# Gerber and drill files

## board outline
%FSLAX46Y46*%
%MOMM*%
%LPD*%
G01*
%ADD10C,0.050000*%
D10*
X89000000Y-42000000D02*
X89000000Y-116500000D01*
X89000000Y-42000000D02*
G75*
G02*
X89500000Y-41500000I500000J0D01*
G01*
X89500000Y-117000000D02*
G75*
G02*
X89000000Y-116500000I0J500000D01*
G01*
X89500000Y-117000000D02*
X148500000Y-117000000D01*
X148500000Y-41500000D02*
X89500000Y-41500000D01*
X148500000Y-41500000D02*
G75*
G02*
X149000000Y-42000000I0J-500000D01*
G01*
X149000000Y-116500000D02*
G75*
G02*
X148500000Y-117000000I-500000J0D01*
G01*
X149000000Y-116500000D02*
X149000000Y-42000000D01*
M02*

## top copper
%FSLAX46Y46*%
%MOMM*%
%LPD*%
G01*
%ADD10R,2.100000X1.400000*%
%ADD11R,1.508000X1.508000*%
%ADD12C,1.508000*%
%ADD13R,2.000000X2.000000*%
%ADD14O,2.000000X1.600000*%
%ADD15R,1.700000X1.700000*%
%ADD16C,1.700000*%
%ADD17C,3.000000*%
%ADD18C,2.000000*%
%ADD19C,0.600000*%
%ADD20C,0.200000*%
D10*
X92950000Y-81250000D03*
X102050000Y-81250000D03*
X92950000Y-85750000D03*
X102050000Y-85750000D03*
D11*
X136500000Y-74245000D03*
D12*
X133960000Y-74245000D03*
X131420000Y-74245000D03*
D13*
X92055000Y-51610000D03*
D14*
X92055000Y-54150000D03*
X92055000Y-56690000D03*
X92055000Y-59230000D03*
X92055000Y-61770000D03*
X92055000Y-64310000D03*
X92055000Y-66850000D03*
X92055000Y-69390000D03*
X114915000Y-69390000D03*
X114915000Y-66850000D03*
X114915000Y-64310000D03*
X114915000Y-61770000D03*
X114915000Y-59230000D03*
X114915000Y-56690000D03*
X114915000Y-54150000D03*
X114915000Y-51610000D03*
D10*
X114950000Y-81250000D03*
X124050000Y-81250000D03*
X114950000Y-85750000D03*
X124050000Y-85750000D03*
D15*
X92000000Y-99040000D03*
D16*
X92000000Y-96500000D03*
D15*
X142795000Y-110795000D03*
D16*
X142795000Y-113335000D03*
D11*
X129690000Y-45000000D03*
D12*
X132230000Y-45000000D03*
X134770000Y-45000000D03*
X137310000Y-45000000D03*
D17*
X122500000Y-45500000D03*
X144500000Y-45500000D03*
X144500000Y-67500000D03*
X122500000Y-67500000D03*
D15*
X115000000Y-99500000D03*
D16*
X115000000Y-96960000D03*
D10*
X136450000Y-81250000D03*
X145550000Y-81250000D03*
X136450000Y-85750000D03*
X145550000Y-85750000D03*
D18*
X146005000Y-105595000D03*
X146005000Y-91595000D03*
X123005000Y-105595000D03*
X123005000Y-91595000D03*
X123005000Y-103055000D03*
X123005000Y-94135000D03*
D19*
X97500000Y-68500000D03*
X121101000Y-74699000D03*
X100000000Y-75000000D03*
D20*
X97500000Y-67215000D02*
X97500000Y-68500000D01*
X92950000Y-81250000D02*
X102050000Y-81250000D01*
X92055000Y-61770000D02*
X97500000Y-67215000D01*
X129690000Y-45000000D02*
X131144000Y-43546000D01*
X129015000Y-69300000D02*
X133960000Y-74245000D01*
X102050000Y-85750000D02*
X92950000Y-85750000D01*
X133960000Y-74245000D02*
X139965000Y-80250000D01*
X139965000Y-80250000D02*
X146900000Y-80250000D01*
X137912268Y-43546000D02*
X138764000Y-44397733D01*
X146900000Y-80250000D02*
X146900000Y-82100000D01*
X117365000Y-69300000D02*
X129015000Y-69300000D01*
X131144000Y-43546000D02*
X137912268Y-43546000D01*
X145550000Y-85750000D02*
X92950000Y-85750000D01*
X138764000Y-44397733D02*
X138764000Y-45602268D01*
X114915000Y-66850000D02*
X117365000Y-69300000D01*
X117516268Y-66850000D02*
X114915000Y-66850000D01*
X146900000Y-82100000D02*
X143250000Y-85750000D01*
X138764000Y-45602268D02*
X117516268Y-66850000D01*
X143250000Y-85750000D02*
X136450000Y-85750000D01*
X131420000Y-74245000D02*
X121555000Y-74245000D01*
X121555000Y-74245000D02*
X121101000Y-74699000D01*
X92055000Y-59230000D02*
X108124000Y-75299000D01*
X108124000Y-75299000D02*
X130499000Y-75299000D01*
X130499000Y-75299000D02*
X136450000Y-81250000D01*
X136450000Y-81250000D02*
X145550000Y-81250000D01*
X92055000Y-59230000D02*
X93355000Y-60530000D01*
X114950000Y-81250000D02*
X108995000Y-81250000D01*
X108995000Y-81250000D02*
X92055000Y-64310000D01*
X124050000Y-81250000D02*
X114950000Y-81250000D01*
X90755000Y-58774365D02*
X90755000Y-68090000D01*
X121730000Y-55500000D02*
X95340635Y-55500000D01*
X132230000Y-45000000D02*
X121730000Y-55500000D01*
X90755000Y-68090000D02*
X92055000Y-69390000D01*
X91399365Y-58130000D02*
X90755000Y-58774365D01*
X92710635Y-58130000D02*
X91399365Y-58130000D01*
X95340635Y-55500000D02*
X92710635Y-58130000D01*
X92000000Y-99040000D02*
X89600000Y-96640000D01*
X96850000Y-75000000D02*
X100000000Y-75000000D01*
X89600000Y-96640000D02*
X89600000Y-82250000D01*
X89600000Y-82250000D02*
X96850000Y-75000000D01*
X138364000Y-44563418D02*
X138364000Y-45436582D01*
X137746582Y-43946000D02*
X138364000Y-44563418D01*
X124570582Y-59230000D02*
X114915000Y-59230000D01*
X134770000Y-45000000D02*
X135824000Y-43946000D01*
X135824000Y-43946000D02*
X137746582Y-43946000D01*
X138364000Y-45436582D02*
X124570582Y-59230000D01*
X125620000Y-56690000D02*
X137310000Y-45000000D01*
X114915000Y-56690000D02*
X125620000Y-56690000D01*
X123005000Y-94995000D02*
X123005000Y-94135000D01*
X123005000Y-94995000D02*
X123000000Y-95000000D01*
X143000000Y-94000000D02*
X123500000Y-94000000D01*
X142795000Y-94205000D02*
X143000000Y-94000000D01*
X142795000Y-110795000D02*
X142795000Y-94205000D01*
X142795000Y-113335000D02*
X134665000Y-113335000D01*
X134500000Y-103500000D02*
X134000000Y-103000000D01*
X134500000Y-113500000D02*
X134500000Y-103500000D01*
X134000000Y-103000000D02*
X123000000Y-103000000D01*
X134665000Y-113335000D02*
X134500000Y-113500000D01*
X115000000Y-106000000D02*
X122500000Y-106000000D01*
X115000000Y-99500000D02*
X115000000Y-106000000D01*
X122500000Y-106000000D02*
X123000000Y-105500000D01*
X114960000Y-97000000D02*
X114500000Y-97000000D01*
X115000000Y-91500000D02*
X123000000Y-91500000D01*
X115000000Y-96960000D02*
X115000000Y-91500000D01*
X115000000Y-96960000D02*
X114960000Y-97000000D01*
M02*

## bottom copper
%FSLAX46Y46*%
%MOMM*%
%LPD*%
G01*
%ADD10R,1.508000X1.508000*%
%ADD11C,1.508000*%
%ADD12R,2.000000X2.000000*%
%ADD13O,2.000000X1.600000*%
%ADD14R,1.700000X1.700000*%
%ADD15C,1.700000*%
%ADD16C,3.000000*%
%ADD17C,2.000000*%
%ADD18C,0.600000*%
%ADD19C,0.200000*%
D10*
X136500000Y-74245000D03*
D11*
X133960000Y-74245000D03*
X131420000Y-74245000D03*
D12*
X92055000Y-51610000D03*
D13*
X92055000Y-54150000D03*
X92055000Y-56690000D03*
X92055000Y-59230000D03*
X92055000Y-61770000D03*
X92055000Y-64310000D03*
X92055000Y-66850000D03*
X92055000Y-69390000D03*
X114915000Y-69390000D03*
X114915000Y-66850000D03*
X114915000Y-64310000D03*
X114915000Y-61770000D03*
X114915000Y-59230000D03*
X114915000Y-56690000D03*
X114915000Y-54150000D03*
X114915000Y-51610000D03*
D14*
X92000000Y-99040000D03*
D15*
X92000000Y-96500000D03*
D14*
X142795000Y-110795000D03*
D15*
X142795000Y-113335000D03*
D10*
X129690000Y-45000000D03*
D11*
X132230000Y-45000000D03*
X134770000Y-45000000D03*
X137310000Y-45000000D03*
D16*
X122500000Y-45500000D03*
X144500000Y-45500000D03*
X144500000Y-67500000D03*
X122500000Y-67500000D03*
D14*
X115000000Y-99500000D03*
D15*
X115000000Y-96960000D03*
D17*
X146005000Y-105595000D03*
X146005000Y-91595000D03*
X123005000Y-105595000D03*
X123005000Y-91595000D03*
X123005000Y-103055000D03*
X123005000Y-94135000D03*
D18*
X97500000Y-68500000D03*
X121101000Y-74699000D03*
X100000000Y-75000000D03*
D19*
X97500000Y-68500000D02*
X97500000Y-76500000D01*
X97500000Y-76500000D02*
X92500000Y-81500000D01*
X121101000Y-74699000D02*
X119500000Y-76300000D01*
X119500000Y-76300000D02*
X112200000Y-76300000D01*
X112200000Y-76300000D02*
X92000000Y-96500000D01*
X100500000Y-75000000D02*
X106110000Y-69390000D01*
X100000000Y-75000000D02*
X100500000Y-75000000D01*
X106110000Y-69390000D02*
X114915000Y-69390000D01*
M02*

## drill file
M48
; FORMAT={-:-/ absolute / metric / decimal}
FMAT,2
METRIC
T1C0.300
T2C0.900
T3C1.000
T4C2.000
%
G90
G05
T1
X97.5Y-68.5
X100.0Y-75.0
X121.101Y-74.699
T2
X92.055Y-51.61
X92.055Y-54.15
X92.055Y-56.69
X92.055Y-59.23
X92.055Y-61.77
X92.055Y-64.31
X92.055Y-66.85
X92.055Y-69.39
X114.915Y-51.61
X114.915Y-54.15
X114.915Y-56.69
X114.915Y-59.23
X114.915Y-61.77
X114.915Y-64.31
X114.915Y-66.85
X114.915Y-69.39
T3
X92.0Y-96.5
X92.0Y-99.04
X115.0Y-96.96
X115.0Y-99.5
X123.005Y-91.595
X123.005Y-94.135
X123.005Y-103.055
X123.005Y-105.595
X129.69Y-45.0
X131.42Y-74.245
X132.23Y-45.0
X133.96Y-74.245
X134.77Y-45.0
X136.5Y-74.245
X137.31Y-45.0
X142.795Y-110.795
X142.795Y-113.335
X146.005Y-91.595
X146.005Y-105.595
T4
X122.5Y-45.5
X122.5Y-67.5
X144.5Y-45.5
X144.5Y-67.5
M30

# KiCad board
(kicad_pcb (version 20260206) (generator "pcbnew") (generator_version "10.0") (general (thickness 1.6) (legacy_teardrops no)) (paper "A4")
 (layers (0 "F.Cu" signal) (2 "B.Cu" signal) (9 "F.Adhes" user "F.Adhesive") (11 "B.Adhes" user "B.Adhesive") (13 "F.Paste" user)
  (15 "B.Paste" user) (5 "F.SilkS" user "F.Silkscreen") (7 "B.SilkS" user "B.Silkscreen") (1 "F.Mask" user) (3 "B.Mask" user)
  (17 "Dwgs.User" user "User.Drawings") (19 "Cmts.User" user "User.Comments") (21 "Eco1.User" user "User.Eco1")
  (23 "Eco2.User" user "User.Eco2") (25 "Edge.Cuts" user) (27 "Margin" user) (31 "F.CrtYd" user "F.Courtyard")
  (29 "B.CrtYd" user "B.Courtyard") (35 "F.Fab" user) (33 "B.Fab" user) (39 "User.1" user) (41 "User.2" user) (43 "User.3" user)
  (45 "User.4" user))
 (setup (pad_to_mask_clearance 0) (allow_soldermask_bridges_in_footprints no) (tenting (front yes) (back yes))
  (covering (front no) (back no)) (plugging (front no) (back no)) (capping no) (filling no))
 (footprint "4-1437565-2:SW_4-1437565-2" (layer "F.Cu") (at 97.5 83.5)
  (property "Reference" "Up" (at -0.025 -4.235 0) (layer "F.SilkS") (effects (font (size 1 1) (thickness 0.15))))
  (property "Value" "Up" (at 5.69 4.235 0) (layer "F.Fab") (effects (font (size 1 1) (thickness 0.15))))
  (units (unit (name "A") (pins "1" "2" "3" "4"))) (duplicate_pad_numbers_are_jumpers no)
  (pad "1" smd rect (at -4.55 -2.25) (size 2.1 1.4) (layers "F.Cu" "F.Mask" "F.Paste") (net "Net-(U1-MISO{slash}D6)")
   (solder_mask_margin 0.102))
  (pad "2" smd rect (at 4.55 -2.25) (size 2.1 1.4) (layers "F.Cu" "F.Mask" "F.Paste") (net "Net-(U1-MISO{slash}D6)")
   (solder_mask_margin 0.102))
  (pad "3" smd rect (at -4.55 2.25) (size 2.1 1.4) (layers "F.Cu" "F.Mask" "F.Paste") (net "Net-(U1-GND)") (solder_mask_margin 0.102))
  (pad "4" smd rect (at 4.55 2.25) (size 2.1 1.4) (layers "F.Cu" "F.Mask" "F.Paste") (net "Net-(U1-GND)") (solder_mask_margin 0.102)))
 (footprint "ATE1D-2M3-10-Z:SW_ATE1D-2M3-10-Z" (layer "F.Cu") (at 133.96 74.245)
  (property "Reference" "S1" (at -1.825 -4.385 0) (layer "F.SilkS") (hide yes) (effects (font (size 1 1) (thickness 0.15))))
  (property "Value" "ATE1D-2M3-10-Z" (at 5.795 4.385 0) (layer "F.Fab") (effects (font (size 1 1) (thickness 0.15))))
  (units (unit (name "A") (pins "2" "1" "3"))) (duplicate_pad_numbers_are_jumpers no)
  (pad "1" thru_hole rect (at 2.54 0) (size 1.508 1.508) (drill 1) (layers "*.Cu" "*.Mask") (remove_unused_layers no)
   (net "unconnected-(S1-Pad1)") (solder_mask_margin 0.102))
  (pad "2" thru_hole circle (at 0 0) (size 1.508 1.508) (drill 1) (layers "*.Cu" "*.Mask") (remove_unused_layers no) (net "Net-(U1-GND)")
   (solder_mask_margin 0.102))
  (pad "3" thru_hole circle (at -2.54 0) (size 1.508 1.508) (drill 1) (layers "*.Cu" "*.Mask") (remove_unused_layers no)
   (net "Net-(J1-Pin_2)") (solder_mask_margin 0.102)))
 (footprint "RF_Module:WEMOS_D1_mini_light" (layer "F.Cu") (at 92.055 51.61)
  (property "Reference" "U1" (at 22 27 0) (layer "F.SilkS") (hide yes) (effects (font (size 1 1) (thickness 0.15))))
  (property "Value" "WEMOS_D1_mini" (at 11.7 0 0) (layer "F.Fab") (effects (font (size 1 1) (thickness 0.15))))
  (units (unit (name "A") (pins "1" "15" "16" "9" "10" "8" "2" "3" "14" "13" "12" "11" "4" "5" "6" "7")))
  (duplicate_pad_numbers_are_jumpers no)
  (pad "1" thru_hole rect (at 0 0) (size 2 2) (drill 0.9) (layers "*.Cu" "*.Mask") (remove_unused_layers no)
   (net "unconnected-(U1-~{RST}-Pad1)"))
  (pad "2" thru_hole oval (at 0 2.54) (size 2 1.6) (drill 0.9) (layers "*.Cu" "*.Mask") (remove_unused_layers no)
   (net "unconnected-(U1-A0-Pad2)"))
  (pad "3" thru_hole oval (at 0 5.08) (size 2 1.6) (drill 0.9) (layers "*.Cu" "*.Mask") (remove_unused_layers no)
   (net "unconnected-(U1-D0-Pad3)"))
  (pad "4" thru_hole oval (at 0 7.62) (size 2 1.6) (drill 0.9) (layers "*.Cu" "*.Mask") (remove_unused_layers no)
   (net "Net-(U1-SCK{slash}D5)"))
  (pad "5" thru_hole oval (at 0 10.16) (size 2 1.6) (drill 0.9) (layers "*.Cu" "*.Mask") (remove_unused_layers no)
   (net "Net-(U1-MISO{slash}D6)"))
  (pad "6" thru_hole oval (at 0 12.7) (size 2 1.6) (drill 0.9) (layers "*.Cu" "*.Mask") (remove_unused_layers no)
   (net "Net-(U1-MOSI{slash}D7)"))
  (pad "7" thru_hole oval (at 0 15.24) (size 2 1.6) (drill 0.9) (layers "*.Cu" "*.Mask") (remove_unused_layers no)
   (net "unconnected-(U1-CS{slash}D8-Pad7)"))
  (pad "8" thru_hole oval (at 0 17.78) (size 2 1.6) (drill 0.9) (layers "*.Cu" "*.Mask") (remove_unused_layers no) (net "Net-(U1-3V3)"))
  (pad "9" thru_hole oval (at 22.86 17.78) (size 2 1.6) (drill 0.9) (layers "*.Cu" "*.Mask") (remove_unused_layers no)
   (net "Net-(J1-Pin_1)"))
  (pad "10" thru_hole oval (at 22.86 15.24) (size 2 1.6) (drill 0.9) (layers "*.Cu" "*.Mask") (remove_unused_layers no) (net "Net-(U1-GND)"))
  (pad "11" thru_hole oval (at 22.86 12.7) (size 2 1.6) (drill 0.9) (layers "*.Cu" "*.Mask") (remove_unused_layers no)
   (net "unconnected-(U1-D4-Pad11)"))
  (pad "12" thru_hole oval (at 22.86 10.16) (size 2 1.6) (drill 0.9) (layers "*.Cu" "*.Mask") (remove_unused_layers no)
   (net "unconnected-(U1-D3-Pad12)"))
  (pad "13" thru_hole oval (at 22.86 7.62) (size 2 1.6) (drill 0.9) (layers "*.Cu" "*.Mask") (remove_unused_layers no)
   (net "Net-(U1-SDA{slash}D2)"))
  (pad "14" thru_hole oval (at 22.86 5.08) (size 2 1.6) (drill 0.9) (layers "*.Cu" "*.Mask") (remove_unused_layers no)
   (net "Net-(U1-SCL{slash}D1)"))
  (pad "15" thru_hole oval (at 22.86 2.54) (size 2 1.6) (drill 0.9) (layers "*.Cu" "*.Mask") (remove_unused_layers no)
   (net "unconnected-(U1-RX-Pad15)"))
  (pad "16" thru_hole oval (at 22.86 0) (size 2 1.6) (drill 0.9) (layers "*.Cu" "*.Mask") (remove_unused_layers no)
   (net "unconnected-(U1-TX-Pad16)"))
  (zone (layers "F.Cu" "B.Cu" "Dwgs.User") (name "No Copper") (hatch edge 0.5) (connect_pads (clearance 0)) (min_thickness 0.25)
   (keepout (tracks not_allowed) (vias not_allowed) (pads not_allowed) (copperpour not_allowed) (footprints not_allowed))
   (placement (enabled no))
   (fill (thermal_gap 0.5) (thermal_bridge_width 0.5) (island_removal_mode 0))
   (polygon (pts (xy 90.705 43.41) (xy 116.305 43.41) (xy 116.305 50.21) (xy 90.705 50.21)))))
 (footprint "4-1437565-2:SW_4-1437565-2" (layer "F.Cu") (at 119.5 83.5)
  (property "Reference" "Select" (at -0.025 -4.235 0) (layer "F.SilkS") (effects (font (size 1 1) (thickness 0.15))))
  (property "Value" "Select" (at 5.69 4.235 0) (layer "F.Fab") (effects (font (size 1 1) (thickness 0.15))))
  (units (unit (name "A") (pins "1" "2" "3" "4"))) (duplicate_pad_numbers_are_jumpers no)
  (pad "1" smd rect (at -4.55 -2.25) (size 2.1 1.4) (layers "F.Cu" "F.Mask" "F.Paste") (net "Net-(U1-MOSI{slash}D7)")
   (solder_mask_margin 0.102))
  (pad "2" smd rect (at 4.55 -2.25) (size 2.1 1.4) (layers "F.Cu" "F.Mask" "F.Paste") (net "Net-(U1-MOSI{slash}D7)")
   (solder_mask_margin 0.102))
  (pad "3" smd rect (at -4.55 2.25) (size 2.1 1.4) (layers "F.Cu" "F.Mask" "F.Paste") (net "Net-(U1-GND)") (solder_mask_margin 0.102))
  (pad "4" smd rect (at 4.55 2.25) (size 2.1 1.4) (layers "F.Cu" "F.Mask" "F.Paste") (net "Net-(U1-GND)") (solder_mask_margin 0.102)))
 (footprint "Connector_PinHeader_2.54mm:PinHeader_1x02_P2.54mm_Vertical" (layer "F.Cu") (at 92 99.04 180)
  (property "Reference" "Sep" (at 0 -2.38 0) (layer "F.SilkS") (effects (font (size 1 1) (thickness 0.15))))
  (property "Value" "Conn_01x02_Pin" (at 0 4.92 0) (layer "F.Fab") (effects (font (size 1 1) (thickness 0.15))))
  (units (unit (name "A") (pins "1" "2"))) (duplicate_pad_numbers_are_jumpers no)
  (pad "1" thru_hole rect (at 0 0 180) (size 1.7 1.7) (drill 1) (layers "*.Cu" "*.Mask") (remove_unused_layers no) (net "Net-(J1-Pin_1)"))
  (pad "2" thru_hole circle (at 0 2.54 180) (size 1.7 1.7) (drill 1) (layers "*.Cu" "*.Mask") (remove_unused_layers no)
   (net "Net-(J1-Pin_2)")))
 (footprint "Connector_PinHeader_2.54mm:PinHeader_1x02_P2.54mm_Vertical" (layer "F.Cu") (at 142.795 110.795)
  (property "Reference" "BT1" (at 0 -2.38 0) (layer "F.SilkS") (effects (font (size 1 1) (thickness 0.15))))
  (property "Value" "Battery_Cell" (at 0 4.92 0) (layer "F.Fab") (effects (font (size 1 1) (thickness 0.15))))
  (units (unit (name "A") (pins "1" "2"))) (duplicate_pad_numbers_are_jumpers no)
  (pad "1" thru_hole rect (at 0 0) (size 1.7 1.7) (drill 1) (layers "*.Cu" "*.Mask") (remove_unused_layers no)
   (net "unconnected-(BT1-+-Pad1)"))
  (pad "2" thru_hole circle (at 0 2.54) (size 1.7 1.7) (drill 1) (layers "*.Cu" "*.Mask") (remove_unused_layers no)
   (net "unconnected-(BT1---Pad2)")))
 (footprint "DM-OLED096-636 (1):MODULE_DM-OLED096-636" (layer "F.Cu") (at 133.5 56.5)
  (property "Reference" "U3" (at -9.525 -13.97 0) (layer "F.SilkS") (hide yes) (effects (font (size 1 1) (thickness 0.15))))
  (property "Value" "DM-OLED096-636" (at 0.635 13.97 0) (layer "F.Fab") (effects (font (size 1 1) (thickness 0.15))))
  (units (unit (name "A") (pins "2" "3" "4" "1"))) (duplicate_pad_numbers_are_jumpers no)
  (pad "1" thru_hole rect (at -3.81 -11.5) (size 1.508 1.508) (drill 1) (layers "*.Cu" "*.Mask") (remove_unused_layers no)
   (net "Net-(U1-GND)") (solder_mask_margin 0.102))
  (pad "2" thru_hole circle (at -1.27 -11.5) (size 1.508 1.508) (drill 1) (layers "*.Cu" "*.Mask") (remove_unused_layers no)
   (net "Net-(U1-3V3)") (solder_mask_margin 0.102))
  (pad "3" thru_hole circle (at 1.27 -11.5) (size 1.508 1.508) (drill 1) (layers "*.Cu" "*.Mask") (remove_unused_layers no)
   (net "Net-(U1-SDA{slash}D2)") (solder_mask_margin 0.102))
  (pad "4" thru_hole circle (at 3.81 -11.5) (size 1.508 1.508) (drill 1) (layers "*.Cu" "*.Mask") (remove_unused_layers no)
   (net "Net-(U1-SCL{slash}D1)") (solder_mask_margin 0.102))
  (pad "S1" thru_hole circle (at -11 -11) (size 3 3) (drill 2) (layers "*.Cu" "*.Mask") (remove_unused_layers no) (solder_mask_margin 0.102))
  (pad "S2" thru_hole circle (at 11 -11) (size 3 3) (drill 2) (layers "*.Cu" "*.Mask") (remove_unused_layers no) (solder_mask_margin 0.102))
  (pad "S3" thru_hole circle (at 11 11) (size 3 3) (drill 2) (layers "*.Cu" "*.Mask") (remove_unused_layers no) (solder_mask_margin 0.102))
  (pad "S4" thru_hole circle (at -11 11) (size 3 3) (drill 2) (layers "*.Cu" "*.Mask") (remove_unused_layers no) (solder_mask_margin 0.102)))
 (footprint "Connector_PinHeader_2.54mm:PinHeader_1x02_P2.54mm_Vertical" (layer "F.Cu") (at 115 99.5 180)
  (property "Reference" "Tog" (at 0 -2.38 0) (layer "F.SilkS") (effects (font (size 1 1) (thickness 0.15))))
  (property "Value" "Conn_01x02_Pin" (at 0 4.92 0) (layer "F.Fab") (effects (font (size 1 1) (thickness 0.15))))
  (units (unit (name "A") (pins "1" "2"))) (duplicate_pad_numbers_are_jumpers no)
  (pad "1" thru_hole rect (at 0 0 180) (size 1.7 1.7) (drill 1) (layers "*.Cu" "*.Mask") (remove_unused_layers no)
   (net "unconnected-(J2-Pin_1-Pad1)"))
  (pad "2" thru_hole circle (at 0 2.54 180) (size 1.7 1.7) (drill 1) (layers "*.Cu" "*.Mask") (remove_unused_layers no)
   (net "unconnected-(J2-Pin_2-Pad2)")))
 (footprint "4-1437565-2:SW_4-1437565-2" (layer "F.Cu") (at 141 83.5)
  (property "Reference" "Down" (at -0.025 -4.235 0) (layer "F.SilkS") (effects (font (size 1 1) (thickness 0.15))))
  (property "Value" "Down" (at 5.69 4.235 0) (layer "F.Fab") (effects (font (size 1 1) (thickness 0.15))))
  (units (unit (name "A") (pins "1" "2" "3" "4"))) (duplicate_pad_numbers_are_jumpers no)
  (pad "1" smd rect (at -4.55 -2.25) (size 2.1 1.4) (layers "F.Cu" "F.Mask" "F.Paste") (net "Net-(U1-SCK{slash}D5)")
   (solder_mask_margin 0.102))
  (pad "2" smd rect (at 4.55 -2.25) (size 2.1 1.4) (layers "F.Cu" "F.Mask" "F.Paste") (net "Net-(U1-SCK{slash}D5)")
   (solder_mask_margin 0.102))
  (pad "3" smd rect (at -4.55 2.25) (size 2.1 1.4) (layers "F.Cu" "F.Mask" "F.Paste") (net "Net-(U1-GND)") (solder_mask_margin 0.102))
  (pad "4" smd rect (at 4.55 2.25) (size 2.1 1.4) (layers "F.Cu" "F.Mask" "F.Paste") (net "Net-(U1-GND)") (solder_mask_margin 0.102)))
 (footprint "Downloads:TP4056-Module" (layer "F.Cu") (at 148.505 89.995 180)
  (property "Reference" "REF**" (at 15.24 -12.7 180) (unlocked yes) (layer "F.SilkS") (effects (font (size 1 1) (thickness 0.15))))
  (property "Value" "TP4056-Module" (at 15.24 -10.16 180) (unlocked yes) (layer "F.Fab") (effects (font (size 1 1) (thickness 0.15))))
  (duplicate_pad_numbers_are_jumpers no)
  (pad "1" thru_hole circle (at 2.5 -15.6 180) (size 2 2) (drill 1) (layers "*.Cu" "*.Mask") (remove_unused_layers no))
  (pad "2" thru_hole circle (at 2.5 -1.6 180) (size 2 2) (drill 1) (layers "*.Cu" "*.Mask") (remove_unused_layers no))
  (pad "3" thru_hole circle (at 25.5 -15.6 180) (size 2 2) (drill 1) (layers "*.Cu" "*.Mask") (remove_unused_layers no))
  (pad "4" thru_hole circle (at 25.5 -1.6 180) (size 2 2) (drill 1) (layers "*.Cu" "*.Mask") (remove_unused_layers no))
  (pad "5" thru_hole circle (at 25.5 -13.06 180) (size 2 2) (drill 1) (layers "*.Cu" "*.Mask") (remove_unused_layers no))
  (pad "6" thru_hole circle (at 25.5 -4.14 180) (size 2 2) (drill 1) (layers "*.Cu" "*.Mask") (remove_unused_layers no)))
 (gr_line (start 89 42) (end 89 116.5) (stroke (width 0.05) (type default)) (layer "Edge.Cuts"))
 (gr_arc (start 89 42) (mid 89.146447 41.646447) (end 89.5 41.5) (stroke (width 0.05) (type default)) (layer "Edge.Cuts"))
 (gr_arc (start 89.5 117) (mid 89.146447 116.853553) (end 89 116.5) (stroke (width 0.05) (type default)) (layer "Edge.Cuts"))
 (gr_line (start 89.5 117) (end 148.5 117) (stroke (width 0.05) (type default)) (layer "Edge.Cuts"))
 (gr_line (start 148.5 41.5) (end 89.5 41.5) (stroke (width 0.05) (type default)) (layer "Edge.Cuts"))
 (gr_arc (start 148.5 41.5) (mid 148.853553 41.646447) (end 149 42) (stroke (width 0.05) (type default)) (layer "Edge.Cuts"))
 (gr_arc (start 149 116.5) (mid 148.853553 116.853553) (end 148.5 117) (stroke (width 0.05) (type default)) (layer "Edge.Cuts"))
 (gr_line (start 149 116.5) (end 149 42) (stroke (width 0.05) (type default)) (layer "Edge.Cuts"))
 (segment (start 97.5 67.215) (end 97.5 68.5) (width 0.2) (layer "F.Cu") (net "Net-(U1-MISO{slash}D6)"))
 (segment (start 92.95 81.25) (end 102.05 81.25) (width 0.2) (layer "F.Cu") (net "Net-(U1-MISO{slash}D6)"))
 (segment (start 92.055 61.77) (end 97.5 67.215) (width 0.2) (layer "F.Cu") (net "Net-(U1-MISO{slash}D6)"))
 (via (at 97.5 68.5) (size 0.6) (drill 0.3) (layers "F.Cu" "B.Cu") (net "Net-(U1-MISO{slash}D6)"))
 (segment (start 97.5 68.5) (end 97.5 76.5) (width 0.2) (layer "B.Cu") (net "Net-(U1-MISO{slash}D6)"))
 (segment (start 97.5 76.5) (end 92.5 81.5) (width 0.2) (layer "B.Cu") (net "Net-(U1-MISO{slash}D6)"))
 (segment (start 129.69 45) (end 131.144 43.546) (width 0.2) (layer "F.Cu") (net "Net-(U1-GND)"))
 (segment (start 129.015 69.3) (end 133.96 74.245) (width 0.2) (layer "F.Cu") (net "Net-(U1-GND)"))
 (segment (start 102.05 85.75) (end 92.95 85.75) (width 0.2) (layer "F.Cu") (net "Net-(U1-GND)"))
 (segment (start 133.96 74.245) (end 139.965 80.25) (width 0.2) (layer "F.Cu") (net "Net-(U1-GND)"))
 (segment (start 139.965 80.25) (end 146.9 80.25) (width 0.2) (layer "F.Cu") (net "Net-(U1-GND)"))
 (segment (start 137.912268 43.546) (end 138.764 44.397733) (width 0.2) (layer "F.Cu") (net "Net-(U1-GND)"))
 (segment (start 146.9 80.25) (end 146.9 82.1) (width 0.2) (layer "F.Cu") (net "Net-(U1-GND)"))
 (segment (start 117.365 69.3) (end 129.015 69.3) (width 0.2) (layer "F.Cu") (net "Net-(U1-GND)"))
 (segment (start 131.144 43.546) (end 137.912268 43.546) (width 0.2) (layer "F.Cu") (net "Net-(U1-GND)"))
 (segment (start 145.55 85.75) (end 92.95 85.75) (width 0.2) (layer "F.Cu") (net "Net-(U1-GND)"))
 (segment (start 138.764 44.397733) (end 138.764 45.602268) (width 0.2) (layer "F.Cu") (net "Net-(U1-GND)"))
 (segment (start 114.915 66.85) (end 117.365 69.3) (width 0.2) (layer "F.Cu") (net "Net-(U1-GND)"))
 (segment (start 117.516268 66.85) (end 114.915 66.85) (width 0.2) (layer "F.Cu") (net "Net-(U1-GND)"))
 (segment (start 146.9 82.1) (end 143.25 85.75) (width 0.2) (layer "F.Cu") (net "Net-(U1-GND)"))
 (segment (start 138.764 45.602268) (end 117.516268 66.85) (width 0.2) (layer "F.Cu") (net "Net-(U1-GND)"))
 (segment (start 143.25 85.75) (end 136.45 85.75) (width 0.2) (layer "F.Cu") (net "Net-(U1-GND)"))
 (segment (start 131.42 74.245) (end 121.555 74.245) (width 0.2) (layer "F.Cu") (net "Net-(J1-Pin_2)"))
 (segment (start 121.555 74.245) (end 121.101 74.699) (width 0.2) (layer "F.Cu") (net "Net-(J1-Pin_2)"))
 (via (at 121.101 74.699) (size 0.6) (drill 0.3) (layers "F.Cu" "B.Cu") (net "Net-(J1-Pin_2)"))
 (segment (start 121.101 74.699) (end 119.5 76.3) (width 0.2) (layer "B.Cu") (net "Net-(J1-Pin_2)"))
 (segment (start 119.5 76.3) (end 112.2 76.3) (width 0.2) (layer "B.Cu") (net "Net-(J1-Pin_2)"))
 (segment (start 112.2 76.3) (end 92 96.5) (width 0.2) (layer "B.Cu") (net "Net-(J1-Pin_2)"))
 (segment (start 92.055 59.23) (end 108.124 75.299) (width 0.2) (layer "F.Cu") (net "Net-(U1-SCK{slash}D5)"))
 (segment (start 108.124 75.299) (end 130.499 75.299) (width 0.2) (layer "F.Cu") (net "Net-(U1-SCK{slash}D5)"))
 (segment (start 130.499 75.299) (end 136.45 81.25) (width 0.2) (layer "F.Cu") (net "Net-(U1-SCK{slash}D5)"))
 (segment (start 136.45 81.25) (end 145.55 81.25) (width 0.2) (layer "F.Cu") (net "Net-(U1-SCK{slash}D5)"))
 (segment (start 92.055 59.23) (end 93.355 60.53) (width 0.2) (layer "F.Cu") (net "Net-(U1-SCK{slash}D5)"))
 (segment (start 114.95 81.25) (end 108.995 81.25) (width 0.2) (layer "F.Cu") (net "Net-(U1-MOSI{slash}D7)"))
 (segment (start 108.995 81.25) (end 92.055 64.31) (width 0.2) (layer "F.Cu") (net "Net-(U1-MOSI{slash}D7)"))
 (segment (start 124.05 81.25) (end 114.95 81.25) (width 0.2) (layer "F.Cu") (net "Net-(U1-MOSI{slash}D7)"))
 (segment (start 90.755 58.774365) (end 90.755 68.09) (width 0.2) (layer "F.Cu") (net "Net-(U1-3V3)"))
 (segment (start 121.73 55.5) (end 95.340635 55.5) (width 0.2) (layer "F.Cu") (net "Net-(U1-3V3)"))
 (segment (start 132.23 45) (end 121.73 55.5) (width 0.2) (layer "F.Cu") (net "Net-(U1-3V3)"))
 (segment (start 90.755 68.09) (end 92.055 69.39) (width 0.2) (layer "F.Cu") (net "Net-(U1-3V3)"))
 (segment (start 91.399365 58.13) (end 90.755 58.774365) (width 0.2) (layer "F.Cu") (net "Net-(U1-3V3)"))
 (segment (start 92.710635 58.13) (end 91.399365 58.13) (width 0.2) (layer "F.Cu") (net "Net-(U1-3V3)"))
 (segment (start 95.340635 55.5) (end 92.710635 58.13) (width 0.2) (layer "F.Cu") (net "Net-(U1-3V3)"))
 (segment (start 92 99.04) (end 89.6 96.64) (width 0.2) (layer "F.Cu") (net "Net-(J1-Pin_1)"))
 (segment (start 96.85 75) (end 100 75) (width 0.2) (layer "F.Cu") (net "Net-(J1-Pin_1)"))
 (segment (start 89.6 96.64) (end 89.6 82.25) (width 0.2) (layer "F.Cu") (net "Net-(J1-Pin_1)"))
 (segment (start 89.6 82.25) (end 96.85 75) (width 0.2) (layer "F.Cu") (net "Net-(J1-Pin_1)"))
 (via (at 100 75) (size 0.6) (drill 0.3) (layers "F.Cu" "B.Cu") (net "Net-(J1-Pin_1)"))
 (segment (start 100.5 75) (end 106.11 69.39) (width 0.2) (layer "B.Cu") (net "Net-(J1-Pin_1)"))
 (segment (start 100 75) (end 100.5 75) (width 0.2) (layer "B.Cu") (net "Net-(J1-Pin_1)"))
 (segment (start 106.11 69.39) (end 114.915 69.39) (width 0.2) (layer "B.Cu") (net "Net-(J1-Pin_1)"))
 (segment (start 138.364 44.563418) (end 138.364 45.436582) (width 0.2) (layer "F.Cu") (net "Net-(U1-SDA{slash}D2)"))
 (segment (start 137.746582 43.946) (end 138.364 44.563418) (width 0.2) (layer "F.Cu") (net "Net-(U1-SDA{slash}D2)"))
 (segment (start 124.570582 59.23) (end 114.915 59.23) (width 0.2) (layer "F.Cu") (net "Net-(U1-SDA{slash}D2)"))
 (segment (start 134.77 45) (end 135.824 43.946) (width 0.2) (layer "F.Cu") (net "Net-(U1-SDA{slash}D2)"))
 (segment (start 135.824 43.946) (end 137.746582 43.946) (width 0.2) (layer "F.Cu") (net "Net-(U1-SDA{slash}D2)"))
 (segment (start 138.364 45.436582) (end 124.570582 59.23) (width 0.2) (layer "F.Cu") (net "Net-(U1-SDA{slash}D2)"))
 (segment (start 125.62 56.69) (end 137.31 45) (width 0.2) (layer "F.Cu") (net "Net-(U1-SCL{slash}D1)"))
 (segment (start 114.915 56.69) (end 125.62 56.69) (width 0.2) (layer "F.Cu") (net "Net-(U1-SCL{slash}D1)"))
 (segment (start 123.005 94.995) (end 123.005 94.135) (width 0.2) (layer "F.Cu") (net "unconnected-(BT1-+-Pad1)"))
 (segment (start 123.005 94.995) (end 123 95) (width 0.2) (layer "F.Cu") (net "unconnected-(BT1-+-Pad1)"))
 (segment (start 143 94) (end 123.5 94) (width 0.2) (layer "F.Cu") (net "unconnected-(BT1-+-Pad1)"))
 (segment (start 142.795 94.205) (end 143 94) (width 0.2) (layer "F.Cu") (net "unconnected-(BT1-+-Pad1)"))
 (segment (start 142.795 110.795) (end 142.795 94.205) (width 0.2) (layer "F.Cu") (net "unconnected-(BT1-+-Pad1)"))
 (segment (start 142.795 113.335) (end 134.665 113.335) (width 0.2) (layer "F.Cu") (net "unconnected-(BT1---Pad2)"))
 (segment (start 134.5 103.5) (end 134 103) (width 0.2) (layer "F.Cu") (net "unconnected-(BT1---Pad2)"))
 (segment (start 134.5 113.5) (end 134.5 103.5) (width 0.2) (layer "F.Cu") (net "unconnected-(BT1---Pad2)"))
 (segment (start 134 103) (end 123 103) (width 0.2) (layer "F.Cu") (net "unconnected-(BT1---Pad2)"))
 (segment (start 134.665 113.335) (end 134.5 113.5) (width 0.2) (layer "F.Cu") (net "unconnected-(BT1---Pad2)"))
 (segment (start 115 106) (end 122.5 106) (width 0.2) (layer "F.Cu") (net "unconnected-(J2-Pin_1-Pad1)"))
 (segment (start 115 99.5) (end 115 106) (width 0.2) (layer "F.Cu") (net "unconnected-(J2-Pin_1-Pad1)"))
 (segment (start 122.5 106) (end 123 105.5) (width 0.2) (layer "F.Cu") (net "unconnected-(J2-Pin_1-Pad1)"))
 (segment (start 114.96 97) (end 114.5 97) (width 0.2) (layer "F.Cu") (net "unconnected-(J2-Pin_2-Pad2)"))
 (segment (start 115 91.5) (end 123 91.5) (width 0.2) (layer "F.Cu") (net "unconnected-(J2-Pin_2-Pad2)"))
 (segment (start 115 96.96) (end 115 91.5) (width 0.2) (layer "F.Cu") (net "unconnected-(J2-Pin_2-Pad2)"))
 (segment (start 115 96.96) (end 114.96 97) (width 0.2) (layer "F.Cu") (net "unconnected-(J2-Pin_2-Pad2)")))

